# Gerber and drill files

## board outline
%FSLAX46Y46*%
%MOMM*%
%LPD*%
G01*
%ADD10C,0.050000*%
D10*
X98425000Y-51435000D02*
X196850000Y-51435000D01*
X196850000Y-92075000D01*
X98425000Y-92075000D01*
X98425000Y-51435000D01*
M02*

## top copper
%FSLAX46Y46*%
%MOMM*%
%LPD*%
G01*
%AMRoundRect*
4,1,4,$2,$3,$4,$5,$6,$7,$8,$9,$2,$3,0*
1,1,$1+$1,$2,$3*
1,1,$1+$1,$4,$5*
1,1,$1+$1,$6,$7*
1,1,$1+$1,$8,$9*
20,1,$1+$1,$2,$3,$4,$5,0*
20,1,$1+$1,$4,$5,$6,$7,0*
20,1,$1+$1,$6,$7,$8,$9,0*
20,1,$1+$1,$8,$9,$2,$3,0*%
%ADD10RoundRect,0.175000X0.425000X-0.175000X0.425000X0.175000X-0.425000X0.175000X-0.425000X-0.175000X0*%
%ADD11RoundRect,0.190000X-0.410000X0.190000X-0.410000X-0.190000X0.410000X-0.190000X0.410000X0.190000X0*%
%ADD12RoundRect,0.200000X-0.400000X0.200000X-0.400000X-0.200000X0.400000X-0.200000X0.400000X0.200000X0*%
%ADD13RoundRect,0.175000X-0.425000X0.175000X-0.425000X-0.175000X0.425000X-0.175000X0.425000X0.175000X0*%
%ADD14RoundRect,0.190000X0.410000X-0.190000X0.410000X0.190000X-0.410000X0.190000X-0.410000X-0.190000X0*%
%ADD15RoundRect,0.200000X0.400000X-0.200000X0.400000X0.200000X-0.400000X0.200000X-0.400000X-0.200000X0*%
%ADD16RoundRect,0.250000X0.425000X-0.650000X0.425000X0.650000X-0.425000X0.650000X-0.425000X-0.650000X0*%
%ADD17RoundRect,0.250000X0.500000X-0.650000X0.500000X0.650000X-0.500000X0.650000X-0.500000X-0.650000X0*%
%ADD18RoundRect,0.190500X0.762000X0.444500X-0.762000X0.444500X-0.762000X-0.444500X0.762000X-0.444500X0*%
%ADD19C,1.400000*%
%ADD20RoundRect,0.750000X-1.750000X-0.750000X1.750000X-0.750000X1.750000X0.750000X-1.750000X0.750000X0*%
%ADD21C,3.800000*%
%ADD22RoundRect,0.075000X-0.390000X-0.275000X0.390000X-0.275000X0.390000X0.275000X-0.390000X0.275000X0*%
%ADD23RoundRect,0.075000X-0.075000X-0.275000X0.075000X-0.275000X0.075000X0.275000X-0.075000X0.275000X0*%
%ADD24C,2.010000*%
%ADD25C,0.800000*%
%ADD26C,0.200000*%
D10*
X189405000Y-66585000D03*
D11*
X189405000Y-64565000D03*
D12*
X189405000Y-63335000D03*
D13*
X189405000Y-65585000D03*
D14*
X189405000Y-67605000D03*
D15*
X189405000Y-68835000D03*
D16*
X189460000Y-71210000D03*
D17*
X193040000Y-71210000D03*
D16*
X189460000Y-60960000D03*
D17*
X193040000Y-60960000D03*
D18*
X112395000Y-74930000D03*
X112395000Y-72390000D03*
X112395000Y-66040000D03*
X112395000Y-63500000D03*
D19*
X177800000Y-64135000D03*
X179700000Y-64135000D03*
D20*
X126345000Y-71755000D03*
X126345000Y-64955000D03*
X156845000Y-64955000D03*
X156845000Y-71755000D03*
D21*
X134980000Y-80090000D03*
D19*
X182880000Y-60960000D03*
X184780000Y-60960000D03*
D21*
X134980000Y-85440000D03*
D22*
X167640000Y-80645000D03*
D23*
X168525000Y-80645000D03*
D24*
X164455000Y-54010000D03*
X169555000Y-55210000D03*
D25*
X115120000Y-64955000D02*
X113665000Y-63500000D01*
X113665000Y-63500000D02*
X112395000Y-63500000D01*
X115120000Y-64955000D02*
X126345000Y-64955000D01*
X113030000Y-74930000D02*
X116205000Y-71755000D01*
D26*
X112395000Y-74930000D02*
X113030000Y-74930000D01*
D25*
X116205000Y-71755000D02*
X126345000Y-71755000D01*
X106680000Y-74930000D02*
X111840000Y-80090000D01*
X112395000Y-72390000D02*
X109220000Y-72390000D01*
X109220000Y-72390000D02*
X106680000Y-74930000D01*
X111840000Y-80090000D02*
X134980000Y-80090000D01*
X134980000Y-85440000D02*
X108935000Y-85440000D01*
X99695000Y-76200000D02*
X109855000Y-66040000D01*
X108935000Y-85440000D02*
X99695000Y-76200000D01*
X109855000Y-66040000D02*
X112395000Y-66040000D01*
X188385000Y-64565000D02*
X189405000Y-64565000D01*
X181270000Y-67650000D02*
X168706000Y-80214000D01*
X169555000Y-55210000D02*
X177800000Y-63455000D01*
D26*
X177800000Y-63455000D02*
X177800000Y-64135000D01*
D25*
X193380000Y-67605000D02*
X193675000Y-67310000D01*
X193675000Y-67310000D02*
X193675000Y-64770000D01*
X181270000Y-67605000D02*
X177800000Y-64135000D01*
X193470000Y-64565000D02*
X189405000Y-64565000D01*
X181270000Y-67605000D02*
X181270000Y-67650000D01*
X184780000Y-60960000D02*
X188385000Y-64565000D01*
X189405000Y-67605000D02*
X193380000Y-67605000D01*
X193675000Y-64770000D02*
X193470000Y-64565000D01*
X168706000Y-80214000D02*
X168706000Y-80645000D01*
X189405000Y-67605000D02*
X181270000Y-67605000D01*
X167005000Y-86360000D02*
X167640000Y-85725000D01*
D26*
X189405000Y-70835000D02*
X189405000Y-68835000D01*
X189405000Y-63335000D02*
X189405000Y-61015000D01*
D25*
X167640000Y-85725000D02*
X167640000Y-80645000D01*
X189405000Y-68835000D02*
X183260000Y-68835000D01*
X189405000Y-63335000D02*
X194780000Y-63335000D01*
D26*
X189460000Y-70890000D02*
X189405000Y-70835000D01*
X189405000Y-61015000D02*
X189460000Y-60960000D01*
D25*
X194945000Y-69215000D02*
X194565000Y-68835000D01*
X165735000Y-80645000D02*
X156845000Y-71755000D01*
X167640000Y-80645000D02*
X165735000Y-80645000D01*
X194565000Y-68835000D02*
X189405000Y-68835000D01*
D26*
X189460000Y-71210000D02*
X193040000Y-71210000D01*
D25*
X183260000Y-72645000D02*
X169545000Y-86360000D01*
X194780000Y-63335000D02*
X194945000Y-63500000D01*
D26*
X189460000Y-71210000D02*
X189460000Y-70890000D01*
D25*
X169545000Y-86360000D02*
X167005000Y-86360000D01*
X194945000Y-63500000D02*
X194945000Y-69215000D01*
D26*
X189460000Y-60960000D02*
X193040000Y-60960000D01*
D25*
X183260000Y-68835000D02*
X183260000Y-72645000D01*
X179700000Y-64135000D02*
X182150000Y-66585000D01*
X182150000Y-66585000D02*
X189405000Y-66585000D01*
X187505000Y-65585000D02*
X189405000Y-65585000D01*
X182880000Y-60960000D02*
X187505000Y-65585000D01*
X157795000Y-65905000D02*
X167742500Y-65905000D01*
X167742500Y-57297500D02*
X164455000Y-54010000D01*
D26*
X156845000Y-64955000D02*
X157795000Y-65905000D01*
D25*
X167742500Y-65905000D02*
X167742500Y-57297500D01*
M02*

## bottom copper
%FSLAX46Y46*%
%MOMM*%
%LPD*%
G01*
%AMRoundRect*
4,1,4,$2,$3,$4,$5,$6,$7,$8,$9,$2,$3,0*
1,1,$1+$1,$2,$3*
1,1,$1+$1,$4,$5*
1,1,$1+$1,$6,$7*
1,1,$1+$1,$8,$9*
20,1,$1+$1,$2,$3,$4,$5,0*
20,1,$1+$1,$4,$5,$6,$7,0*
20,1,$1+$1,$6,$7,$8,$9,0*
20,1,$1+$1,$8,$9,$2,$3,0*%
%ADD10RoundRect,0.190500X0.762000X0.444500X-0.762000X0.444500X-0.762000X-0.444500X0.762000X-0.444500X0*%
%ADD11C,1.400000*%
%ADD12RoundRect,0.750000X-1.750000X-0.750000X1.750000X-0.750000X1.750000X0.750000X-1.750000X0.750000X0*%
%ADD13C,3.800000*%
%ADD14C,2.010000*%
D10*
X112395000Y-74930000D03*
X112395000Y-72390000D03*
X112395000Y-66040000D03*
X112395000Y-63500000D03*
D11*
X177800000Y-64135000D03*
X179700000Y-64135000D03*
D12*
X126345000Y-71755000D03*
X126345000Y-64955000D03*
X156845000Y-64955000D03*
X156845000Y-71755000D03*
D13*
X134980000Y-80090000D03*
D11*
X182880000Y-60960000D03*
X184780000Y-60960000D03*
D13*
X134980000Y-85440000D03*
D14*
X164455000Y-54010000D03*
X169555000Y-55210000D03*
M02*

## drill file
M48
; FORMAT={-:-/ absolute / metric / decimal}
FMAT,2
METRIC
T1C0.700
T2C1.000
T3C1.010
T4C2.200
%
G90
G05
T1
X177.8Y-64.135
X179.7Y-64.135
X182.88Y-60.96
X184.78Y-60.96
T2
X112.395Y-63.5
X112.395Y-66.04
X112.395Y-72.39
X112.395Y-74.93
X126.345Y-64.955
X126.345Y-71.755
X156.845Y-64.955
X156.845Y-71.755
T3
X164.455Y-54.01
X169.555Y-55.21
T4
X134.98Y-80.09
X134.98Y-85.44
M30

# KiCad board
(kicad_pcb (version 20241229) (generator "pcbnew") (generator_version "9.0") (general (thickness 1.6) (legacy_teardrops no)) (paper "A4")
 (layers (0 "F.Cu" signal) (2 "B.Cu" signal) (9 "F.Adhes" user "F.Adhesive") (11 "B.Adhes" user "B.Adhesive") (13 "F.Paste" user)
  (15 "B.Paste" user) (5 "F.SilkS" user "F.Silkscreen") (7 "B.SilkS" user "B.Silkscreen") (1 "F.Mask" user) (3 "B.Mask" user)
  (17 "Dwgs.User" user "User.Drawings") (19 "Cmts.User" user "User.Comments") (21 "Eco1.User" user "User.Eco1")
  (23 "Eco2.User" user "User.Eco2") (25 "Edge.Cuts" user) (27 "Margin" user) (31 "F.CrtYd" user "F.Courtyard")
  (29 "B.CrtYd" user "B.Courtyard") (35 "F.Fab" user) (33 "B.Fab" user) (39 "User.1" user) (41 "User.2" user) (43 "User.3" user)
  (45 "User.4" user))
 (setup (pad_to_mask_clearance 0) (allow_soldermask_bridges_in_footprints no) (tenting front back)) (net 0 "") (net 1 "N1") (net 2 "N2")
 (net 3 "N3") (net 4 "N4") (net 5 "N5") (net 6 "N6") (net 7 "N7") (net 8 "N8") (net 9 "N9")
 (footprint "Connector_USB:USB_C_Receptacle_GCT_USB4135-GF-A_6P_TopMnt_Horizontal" (layer "F.Cu") (at 192.4375 66.085 90)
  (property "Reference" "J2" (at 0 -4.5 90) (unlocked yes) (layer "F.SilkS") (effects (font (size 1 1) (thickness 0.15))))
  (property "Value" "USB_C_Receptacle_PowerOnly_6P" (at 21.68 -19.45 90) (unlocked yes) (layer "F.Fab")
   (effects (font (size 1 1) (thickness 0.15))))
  (pad "A5" smd roundrect (at -0.5 -3.0325 90) (size 0.7 1.2) (layers "F.Cu" "F.Mask" "F.Paste") (roundrect_rratio 0.25) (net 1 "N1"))
  (pad "A9" smd roundrect (at 1.52 -3.0325 270) (size 0.76 1.2) (layers "F.Cu" "F.Mask" "F.Paste") (roundrect_rratio 0.25) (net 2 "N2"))
  (pad "A12" smd roundrect (at 2.75 -3.0325 270) (size 0.8 1.2) (layers "F.Cu" "F.Mask" "F.Paste") (roundrect_rratio 0.25) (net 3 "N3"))
  (pad "B5" smd roundrect (at 0.5 -3.0325 270) (size 0.7 1.2) (layers "F.Cu" "F.Mask" "F.Paste") (roundrect_rratio 0.25) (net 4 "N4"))
  (pad "B9" smd roundrect (at -1.52 -3.0325 90) (size 0.76 1.2) (layers "F.Cu" "F.Mask" "F.Paste") (roundrect_rratio 0.25) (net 2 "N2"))
  (pad "B12" smd roundrect (at -2.75 -3.0325 90) (size 0.8 1.2) (layers "F.Cu" "F.Mask" "F.Paste") (roundrect_rratio 0.25) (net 3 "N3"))
  (pad "S1" smd roundrect (at -5.125 -2.9775 90) (size 1.8 1.35) (layers "F.Cu" "F.Mask" "F.Paste") (roundrect_rratio 0.1851851852)
   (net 3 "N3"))
  (pad "S1" smd roundrect (at -5.125 0.6025 90) (size 1.8 1.5) (layers "F.Cu" "F.Mask" "F.Paste") (roundrect_rratio 0.1666666667)
   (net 3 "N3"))
  (pad "S1" smd roundrect (at 5.125 -2.9775 90) (size 1.8 1.35) (layers "F.Cu" "F.Mask" "F.Paste") (roundrect_rratio 0.1851851852)
   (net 3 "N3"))
  (pad "S1" smd roundrect (at 5.125 0.6025 90) (size 1.8 1.5) (layers "F.Cu" "F.Mask" "F.Paste") (roundrect_rratio 0.1666666667)
   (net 3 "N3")))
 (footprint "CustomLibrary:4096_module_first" (layer "F.Cu") (at 120.015 60.96 180)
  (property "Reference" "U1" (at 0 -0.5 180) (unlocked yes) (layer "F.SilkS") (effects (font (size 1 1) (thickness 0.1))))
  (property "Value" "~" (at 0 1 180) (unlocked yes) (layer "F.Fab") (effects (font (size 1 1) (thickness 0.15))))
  (pad "1" thru_hole roundrect (at 7.62 -13.97 180) (size 1.905 1.27) (drill 1) (layers "*.Cu" "*.Mask") (remove_unused_layers no)
   (roundrect_rratio 0.15) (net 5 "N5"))
  (pad "2" thru_hole roundrect (at 7.62 -11.43 180) (size 1.905 1.27) (drill 1) (layers "*.Cu" "*.Mask") (remove_unused_layers no)
   (roundrect_rratio 0.15) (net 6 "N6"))
  (pad "3" thru_hole roundrect (at 7.62 -5.08 180) (size 1.905 1.27) (drill 1) (layers "*.Cu" "*.Mask") (remove_unused_layers no)
   (roundrect_rratio 0.15) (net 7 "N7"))
  (pad "4" thru_hole roundrect (at 7.62 -2.54 180) (size 1.905 1.27) (drill 1) (layers "*.Cu" "*.Mask") (remove_unused_layers no)
   (roundrect_rratio 0.15) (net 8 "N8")))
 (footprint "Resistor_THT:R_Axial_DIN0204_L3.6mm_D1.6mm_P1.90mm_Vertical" (layer "F.Cu") (at 177.8 64.135)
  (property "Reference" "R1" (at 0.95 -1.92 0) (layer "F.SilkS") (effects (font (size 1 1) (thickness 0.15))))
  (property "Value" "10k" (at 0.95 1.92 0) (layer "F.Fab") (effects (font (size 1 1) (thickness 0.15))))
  (pad "1" thru_hole circle (at 0 0) (size 1.4 1.4) (drill 0.7) (layers "*.Cu" "*.Mask") (remove_unused_layers no) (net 2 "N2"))
  (pad "2" thru_hole circle (at 1.9 0) (size 1.4 1.4) (drill 0.7) (layers "*.Cu" "*.Mask") (remove_unused_layers no) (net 1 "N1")))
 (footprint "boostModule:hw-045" (layer "F.Cu") (at 141.345 68.855)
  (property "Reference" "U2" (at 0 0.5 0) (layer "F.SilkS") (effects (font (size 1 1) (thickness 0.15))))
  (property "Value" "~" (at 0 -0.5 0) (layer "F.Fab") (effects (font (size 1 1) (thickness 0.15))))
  (pad "1" thru_hole roundrect (at -15 2.9) (size 5 3) (drill 1) (layers "*.Cu" "*.Mask") (remove_unused_layers no) (roundrect_rratio 0.25)
   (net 5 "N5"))
  (pad "2" thru_hole roundrect (at -15 -3.9) (size 5 3) (drill 1) (layers "*.Cu" "*.Mask") (remove_unused_layers no) (roundrect_rratio 0.25)
   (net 8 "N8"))
  (pad "3" thru_hole roundrect (at 15.5 -3.9) (size 5 3) (drill 1) (layers "*.Cu" "*.Mask") (remove_unused_layers no)
   (roundrect_rratio 0.25) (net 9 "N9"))
  (pad "4" thru_hole roundrect (at 15.5 2.9) (size 5 3) (drill 1) (layers "*.Cu" "*.Mask") (remove_unused_layers no) (roundrect_rratio 0.25)
   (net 3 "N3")))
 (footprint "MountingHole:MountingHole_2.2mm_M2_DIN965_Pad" (layer "F.Cu") (at 134.98 80.09)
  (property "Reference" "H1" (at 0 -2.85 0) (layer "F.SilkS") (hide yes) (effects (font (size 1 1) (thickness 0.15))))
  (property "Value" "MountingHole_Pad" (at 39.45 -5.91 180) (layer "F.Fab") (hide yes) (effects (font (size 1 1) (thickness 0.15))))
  (pad "1" thru_hole circle (at 0 0) (size 3.8 3.8) (drill 2.2) (layers "*.Cu" "*.Mask") (remove_unused_layers no) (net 6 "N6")
   (zone_connect 2)))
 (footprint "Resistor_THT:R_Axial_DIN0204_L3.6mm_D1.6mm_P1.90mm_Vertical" (layer "F.Cu") (at 182.88 60.96)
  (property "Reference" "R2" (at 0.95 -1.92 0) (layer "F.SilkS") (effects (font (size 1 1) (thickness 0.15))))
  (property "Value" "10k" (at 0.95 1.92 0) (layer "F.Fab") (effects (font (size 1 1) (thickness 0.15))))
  (pad "1" thru_hole circle (at 0 0) (size 1.4 1.4) (drill 0.7) (layers "*.Cu" "*.Mask") (remove_unused_layers no) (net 4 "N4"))
  (pad "2" thru_hole circle (at 1.9 0) (size 1.4 1.4) (drill 0.7) (layers "*.Cu" "*.Mask") (remove_unused_layers no) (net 2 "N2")))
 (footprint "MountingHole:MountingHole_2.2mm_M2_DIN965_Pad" (layer "F.Cu") (at 134.98 85.44)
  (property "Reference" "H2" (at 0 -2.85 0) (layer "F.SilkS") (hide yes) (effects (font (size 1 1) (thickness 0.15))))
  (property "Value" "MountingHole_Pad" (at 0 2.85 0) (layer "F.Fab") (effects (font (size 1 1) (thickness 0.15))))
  (pad "1" thru_hole circle (at 0 0) (size 3.8 3.8) (drill 2.2) (layers "*.Cu" "*.Mask") (remove_unused_layers no) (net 7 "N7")
   (zone_connect 2)))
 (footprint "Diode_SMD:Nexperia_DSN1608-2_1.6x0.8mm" (layer "F.Cu") (at 167.925 80.645)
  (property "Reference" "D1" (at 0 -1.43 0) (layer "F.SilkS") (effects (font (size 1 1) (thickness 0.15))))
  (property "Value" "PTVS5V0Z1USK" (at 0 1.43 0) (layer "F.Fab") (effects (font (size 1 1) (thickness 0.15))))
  (pad "1" smd roundrect (at -0.285 0) (size 0.93 0.7) (layers "F.Cu" "F.Mask" "F.Paste") (roundrect_rratio 0.1071428571) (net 3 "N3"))
  (pad "2" smd roundrect (at 0.6 0) (size 0.3 0.7) (layers "F.Cu" "F.Mask" "F.Paste") (roundrect_rratio 0.25) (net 2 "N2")))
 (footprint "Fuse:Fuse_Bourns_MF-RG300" (layer "F.Cu") (at 164.455 54.01)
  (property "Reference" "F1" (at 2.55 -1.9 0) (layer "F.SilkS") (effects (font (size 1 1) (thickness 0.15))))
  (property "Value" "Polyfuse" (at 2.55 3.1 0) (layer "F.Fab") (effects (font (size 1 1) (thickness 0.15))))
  (pad "1" thru_hole circle (at 0 0) (size 2.01 2.01) (drill 1.01) (layers "*.Cu" "*.Mask") (remove_unused_layers no) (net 9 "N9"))
  (pad "2" thru_hole circle (at 5.1 1.2) (size 2.01 2.01) (drill 1.01) (layers "*.Cu" "*.Mask") (remove_unused_layers no) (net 2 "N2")))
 (gr_rect (start 98.425 51.435) (end 196.85 92.075) (stroke (width 0.05) (type default)) (fill no) (layer "Edge.Cuts"))
 (segment (start 115.12 64.955) (end 113.665 63.5) (width 0.8) (layer "F.Cu") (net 8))
 (segment (start 113.665 63.5) (end 112.395 63.5) (width 0.8) (layer "F.Cu") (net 8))
 (segment (start 115.12 64.955) (end 126.345 64.955) (width 0.8) (layer "F.Cu") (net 8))
 (segment (start 113.03 74.93) (end 116.205 71.755) (width 0.8) (layer "F.Cu") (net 5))
 (segment (start 112.395 74.93) (end 113.03 74.93) (width 0.2) (layer "F.Cu") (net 5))
 (segment (start 116.205 71.755) (end 126.345 71.755) (width 0.8) (layer "F.Cu") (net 5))
 (segment (start 106.68 74.93) (end 111.84 80.09) (width 0.8) (layer "F.Cu") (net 6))
 (segment (start 112.395 72.39) (end 109.22 72.39) (width 0.8) (layer "F.Cu") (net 6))
 (segment (start 109.22 72.39) (end 106.68 74.93) (width 0.8) (layer "F.Cu") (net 6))
 (segment (start 111.84 80.09) (end 134.98 80.09) (width 0.8) (layer "F.Cu") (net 6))
 (segment (start 134.98 85.44) (end 108.935 85.44) (width 0.8) (layer "F.Cu") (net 7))
 (segment (start 99.695 76.2) (end 109.855 66.04) (width 0.8) (layer "F.Cu") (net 7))
 (segment (start 108.935 85.44) (end 99.695 76.2) (width 0.8) (layer "F.Cu") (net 7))
 (segment (start 109.855 66.04) (end 112.395 66.04) (width 0.8) (layer "F.Cu") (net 7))
 (segment (start 188.385 64.565) (end 189.405 64.565) (width 0.8) (layer "F.Cu") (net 2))
 (segment (start 181.27 67.65) (end 168.706 80.214) (width 0.8) (layer "F.Cu") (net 2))
 (segment (start 169.555 55.21) (end 177.8 63.455) (width 0.8) (layer "F.Cu") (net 2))
 (segment (start 177.8 63.455) (end 177.8 64.135) (width 0.2) (layer "F.Cu") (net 2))
 (segment (start 193.38 67.605) (end 193.675 67.31) (width 0.8) (layer "F.Cu") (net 2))
 (segment (start 193.675 67.31) (end 193.675 64.77) (width 0.8) (layer "F.Cu") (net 2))
 (segment (start 181.27 67.605) (end 177.8 64.135) (width 0.8) (layer "F.Cu") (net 2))
 (segment (start 193.47 64.565) (end 189.405 64.565) (width 0.8) (layer "F.Cu") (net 2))
 (segment (start 181.27 67.605) (end 181.27 67.65) (width 0.8) (layer "F.Cu") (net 2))
 (segment (start 184.78 60.96) (end 188.385 64.565) (width 0.8) (layer "F.Cu") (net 2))
 (segment (start 189.405 67.605) (end 193.38 67.605) (width 0.8) (layer "F.Cu") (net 2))
 (segment (start 193.675 64.77) (end 193.47 64.565) (width 0.8) (layer "F.Cu") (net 2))
 (segment (start 168.706 80.214) (end 168.706 80.645) (width 0.8) (layer "F.Cu") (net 2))
 (segment (start 189.405 67.605) (end 181.27 67.605) (width 0.8) (layer "F.Cu") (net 2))
 (segment (start 167.005 86.36) (end 167.64 85.725) (width 0.8) (layer "F.Cu") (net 3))
 (segment (start 189.405 70.835) (end 189.405 68.835) (width 0.2) (layer "F.Cu") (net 3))
 (segment (start 189.405 63.335) (end 189.405 61.015) (width 0.2) (layer "F.Cu") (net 3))
 (segment (start 167.64 85.725) (end 167.64 80.645) (width 0.8) (layer "F.Cu") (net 3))
 (segment (start 189.405 68.835) (end 183.26 68.835) (width 0.8) (layer "F.Cu") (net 3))
 (segment (start 189.405 63.335) (end 194.78 63.335) (width 0.8) (layer "F.Cu") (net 3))
 (segment (start 189.46 70.89) (end 189.405 70.835) (width 0.2) (layer "F.Cu") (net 3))
 (segment (start 189.405 61.015) (end 189.46 60.96) (width 0.2) (layer "F.Cu") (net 3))
 (segment (start 194.945 69.215) (end 194.565 68.835) (width 0.8) (layer "F.Cu") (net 3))
 (segment (start 165.735 80.645) (end 156.845 71.755) (width 0.8) (layer "F.Cu") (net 3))
 (segment (start 167.64 80.645) (end 165.735 80.645) (width 0.8) (layer "F.Cu") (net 3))
 (segment (start 194.565 68.835) (end 189.405 68.835) (width 0.8) (layer "F.Cu") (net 3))
 (segment (start 189.46 71.21) (end 193.04 71.21) (width 0.2) (layer "F.Cu") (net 3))
 (segment (start 183.26 72.645) (end 169.545 86.36) (width 0.8) (layer "F.Cu") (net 3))
 (segment (start 194.78 63.335) (end 194.945 63.5) (width 0.8) (layer "F.Cu") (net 3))
 (segment (start 189.46 71.21) (end 189.46 70.89) (width 0.2) (layer "F.Cu") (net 3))
 (segment (start 169.545 86.36) (end 167.005 86.36) (width 0.8) (layer "F.Cu") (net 3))
 (segment (start 194.945 63.5) (end 194.945 69.215) (width 0.8) (layer "F.Cu") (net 3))
 (segment (start 189.46 60.96) (end 193.04 60.96) (width 0.2) (layer "F.Cu") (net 3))
 (segment (start 183.26 68.835) (end 183.26 72.645) (width 0.8) (layer "F.Cu") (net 3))
 (segment (start 179.7 64.135) (end 182.15 66.585) (width 0.8) (layer "F.Cu") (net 1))
 (segment (start 182.15 66.585) (end 189.405 66.585) (width 0.8) (layer "F.Cu") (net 1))
 (segment (start 187.505 65.585) (end 189.405 65.585) (width 0.8) (layer "F.Cu") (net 4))
 (segment (start 182.88 60.96) (end 187.505 65.585) (width 0.8) (layer "F.Cu") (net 4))
 (segment (start 157.795 65.905) (end 167.7425 65.905) (width 0.8) (layer "F.Cu") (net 9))
 (segment (start 167.7425 57.2975) (end 164.455 54.01) (width 0.8) (layer "F.Cu") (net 9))
 (segment (start 156.845 64.955) (end 157.795 65.905) (width 0.2) (layer "F.Cu") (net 9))
 (segment (start 167.7425 65.905) (end 167.7425 57.2975) (width 0.8) (layer "F.Cu") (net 9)))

